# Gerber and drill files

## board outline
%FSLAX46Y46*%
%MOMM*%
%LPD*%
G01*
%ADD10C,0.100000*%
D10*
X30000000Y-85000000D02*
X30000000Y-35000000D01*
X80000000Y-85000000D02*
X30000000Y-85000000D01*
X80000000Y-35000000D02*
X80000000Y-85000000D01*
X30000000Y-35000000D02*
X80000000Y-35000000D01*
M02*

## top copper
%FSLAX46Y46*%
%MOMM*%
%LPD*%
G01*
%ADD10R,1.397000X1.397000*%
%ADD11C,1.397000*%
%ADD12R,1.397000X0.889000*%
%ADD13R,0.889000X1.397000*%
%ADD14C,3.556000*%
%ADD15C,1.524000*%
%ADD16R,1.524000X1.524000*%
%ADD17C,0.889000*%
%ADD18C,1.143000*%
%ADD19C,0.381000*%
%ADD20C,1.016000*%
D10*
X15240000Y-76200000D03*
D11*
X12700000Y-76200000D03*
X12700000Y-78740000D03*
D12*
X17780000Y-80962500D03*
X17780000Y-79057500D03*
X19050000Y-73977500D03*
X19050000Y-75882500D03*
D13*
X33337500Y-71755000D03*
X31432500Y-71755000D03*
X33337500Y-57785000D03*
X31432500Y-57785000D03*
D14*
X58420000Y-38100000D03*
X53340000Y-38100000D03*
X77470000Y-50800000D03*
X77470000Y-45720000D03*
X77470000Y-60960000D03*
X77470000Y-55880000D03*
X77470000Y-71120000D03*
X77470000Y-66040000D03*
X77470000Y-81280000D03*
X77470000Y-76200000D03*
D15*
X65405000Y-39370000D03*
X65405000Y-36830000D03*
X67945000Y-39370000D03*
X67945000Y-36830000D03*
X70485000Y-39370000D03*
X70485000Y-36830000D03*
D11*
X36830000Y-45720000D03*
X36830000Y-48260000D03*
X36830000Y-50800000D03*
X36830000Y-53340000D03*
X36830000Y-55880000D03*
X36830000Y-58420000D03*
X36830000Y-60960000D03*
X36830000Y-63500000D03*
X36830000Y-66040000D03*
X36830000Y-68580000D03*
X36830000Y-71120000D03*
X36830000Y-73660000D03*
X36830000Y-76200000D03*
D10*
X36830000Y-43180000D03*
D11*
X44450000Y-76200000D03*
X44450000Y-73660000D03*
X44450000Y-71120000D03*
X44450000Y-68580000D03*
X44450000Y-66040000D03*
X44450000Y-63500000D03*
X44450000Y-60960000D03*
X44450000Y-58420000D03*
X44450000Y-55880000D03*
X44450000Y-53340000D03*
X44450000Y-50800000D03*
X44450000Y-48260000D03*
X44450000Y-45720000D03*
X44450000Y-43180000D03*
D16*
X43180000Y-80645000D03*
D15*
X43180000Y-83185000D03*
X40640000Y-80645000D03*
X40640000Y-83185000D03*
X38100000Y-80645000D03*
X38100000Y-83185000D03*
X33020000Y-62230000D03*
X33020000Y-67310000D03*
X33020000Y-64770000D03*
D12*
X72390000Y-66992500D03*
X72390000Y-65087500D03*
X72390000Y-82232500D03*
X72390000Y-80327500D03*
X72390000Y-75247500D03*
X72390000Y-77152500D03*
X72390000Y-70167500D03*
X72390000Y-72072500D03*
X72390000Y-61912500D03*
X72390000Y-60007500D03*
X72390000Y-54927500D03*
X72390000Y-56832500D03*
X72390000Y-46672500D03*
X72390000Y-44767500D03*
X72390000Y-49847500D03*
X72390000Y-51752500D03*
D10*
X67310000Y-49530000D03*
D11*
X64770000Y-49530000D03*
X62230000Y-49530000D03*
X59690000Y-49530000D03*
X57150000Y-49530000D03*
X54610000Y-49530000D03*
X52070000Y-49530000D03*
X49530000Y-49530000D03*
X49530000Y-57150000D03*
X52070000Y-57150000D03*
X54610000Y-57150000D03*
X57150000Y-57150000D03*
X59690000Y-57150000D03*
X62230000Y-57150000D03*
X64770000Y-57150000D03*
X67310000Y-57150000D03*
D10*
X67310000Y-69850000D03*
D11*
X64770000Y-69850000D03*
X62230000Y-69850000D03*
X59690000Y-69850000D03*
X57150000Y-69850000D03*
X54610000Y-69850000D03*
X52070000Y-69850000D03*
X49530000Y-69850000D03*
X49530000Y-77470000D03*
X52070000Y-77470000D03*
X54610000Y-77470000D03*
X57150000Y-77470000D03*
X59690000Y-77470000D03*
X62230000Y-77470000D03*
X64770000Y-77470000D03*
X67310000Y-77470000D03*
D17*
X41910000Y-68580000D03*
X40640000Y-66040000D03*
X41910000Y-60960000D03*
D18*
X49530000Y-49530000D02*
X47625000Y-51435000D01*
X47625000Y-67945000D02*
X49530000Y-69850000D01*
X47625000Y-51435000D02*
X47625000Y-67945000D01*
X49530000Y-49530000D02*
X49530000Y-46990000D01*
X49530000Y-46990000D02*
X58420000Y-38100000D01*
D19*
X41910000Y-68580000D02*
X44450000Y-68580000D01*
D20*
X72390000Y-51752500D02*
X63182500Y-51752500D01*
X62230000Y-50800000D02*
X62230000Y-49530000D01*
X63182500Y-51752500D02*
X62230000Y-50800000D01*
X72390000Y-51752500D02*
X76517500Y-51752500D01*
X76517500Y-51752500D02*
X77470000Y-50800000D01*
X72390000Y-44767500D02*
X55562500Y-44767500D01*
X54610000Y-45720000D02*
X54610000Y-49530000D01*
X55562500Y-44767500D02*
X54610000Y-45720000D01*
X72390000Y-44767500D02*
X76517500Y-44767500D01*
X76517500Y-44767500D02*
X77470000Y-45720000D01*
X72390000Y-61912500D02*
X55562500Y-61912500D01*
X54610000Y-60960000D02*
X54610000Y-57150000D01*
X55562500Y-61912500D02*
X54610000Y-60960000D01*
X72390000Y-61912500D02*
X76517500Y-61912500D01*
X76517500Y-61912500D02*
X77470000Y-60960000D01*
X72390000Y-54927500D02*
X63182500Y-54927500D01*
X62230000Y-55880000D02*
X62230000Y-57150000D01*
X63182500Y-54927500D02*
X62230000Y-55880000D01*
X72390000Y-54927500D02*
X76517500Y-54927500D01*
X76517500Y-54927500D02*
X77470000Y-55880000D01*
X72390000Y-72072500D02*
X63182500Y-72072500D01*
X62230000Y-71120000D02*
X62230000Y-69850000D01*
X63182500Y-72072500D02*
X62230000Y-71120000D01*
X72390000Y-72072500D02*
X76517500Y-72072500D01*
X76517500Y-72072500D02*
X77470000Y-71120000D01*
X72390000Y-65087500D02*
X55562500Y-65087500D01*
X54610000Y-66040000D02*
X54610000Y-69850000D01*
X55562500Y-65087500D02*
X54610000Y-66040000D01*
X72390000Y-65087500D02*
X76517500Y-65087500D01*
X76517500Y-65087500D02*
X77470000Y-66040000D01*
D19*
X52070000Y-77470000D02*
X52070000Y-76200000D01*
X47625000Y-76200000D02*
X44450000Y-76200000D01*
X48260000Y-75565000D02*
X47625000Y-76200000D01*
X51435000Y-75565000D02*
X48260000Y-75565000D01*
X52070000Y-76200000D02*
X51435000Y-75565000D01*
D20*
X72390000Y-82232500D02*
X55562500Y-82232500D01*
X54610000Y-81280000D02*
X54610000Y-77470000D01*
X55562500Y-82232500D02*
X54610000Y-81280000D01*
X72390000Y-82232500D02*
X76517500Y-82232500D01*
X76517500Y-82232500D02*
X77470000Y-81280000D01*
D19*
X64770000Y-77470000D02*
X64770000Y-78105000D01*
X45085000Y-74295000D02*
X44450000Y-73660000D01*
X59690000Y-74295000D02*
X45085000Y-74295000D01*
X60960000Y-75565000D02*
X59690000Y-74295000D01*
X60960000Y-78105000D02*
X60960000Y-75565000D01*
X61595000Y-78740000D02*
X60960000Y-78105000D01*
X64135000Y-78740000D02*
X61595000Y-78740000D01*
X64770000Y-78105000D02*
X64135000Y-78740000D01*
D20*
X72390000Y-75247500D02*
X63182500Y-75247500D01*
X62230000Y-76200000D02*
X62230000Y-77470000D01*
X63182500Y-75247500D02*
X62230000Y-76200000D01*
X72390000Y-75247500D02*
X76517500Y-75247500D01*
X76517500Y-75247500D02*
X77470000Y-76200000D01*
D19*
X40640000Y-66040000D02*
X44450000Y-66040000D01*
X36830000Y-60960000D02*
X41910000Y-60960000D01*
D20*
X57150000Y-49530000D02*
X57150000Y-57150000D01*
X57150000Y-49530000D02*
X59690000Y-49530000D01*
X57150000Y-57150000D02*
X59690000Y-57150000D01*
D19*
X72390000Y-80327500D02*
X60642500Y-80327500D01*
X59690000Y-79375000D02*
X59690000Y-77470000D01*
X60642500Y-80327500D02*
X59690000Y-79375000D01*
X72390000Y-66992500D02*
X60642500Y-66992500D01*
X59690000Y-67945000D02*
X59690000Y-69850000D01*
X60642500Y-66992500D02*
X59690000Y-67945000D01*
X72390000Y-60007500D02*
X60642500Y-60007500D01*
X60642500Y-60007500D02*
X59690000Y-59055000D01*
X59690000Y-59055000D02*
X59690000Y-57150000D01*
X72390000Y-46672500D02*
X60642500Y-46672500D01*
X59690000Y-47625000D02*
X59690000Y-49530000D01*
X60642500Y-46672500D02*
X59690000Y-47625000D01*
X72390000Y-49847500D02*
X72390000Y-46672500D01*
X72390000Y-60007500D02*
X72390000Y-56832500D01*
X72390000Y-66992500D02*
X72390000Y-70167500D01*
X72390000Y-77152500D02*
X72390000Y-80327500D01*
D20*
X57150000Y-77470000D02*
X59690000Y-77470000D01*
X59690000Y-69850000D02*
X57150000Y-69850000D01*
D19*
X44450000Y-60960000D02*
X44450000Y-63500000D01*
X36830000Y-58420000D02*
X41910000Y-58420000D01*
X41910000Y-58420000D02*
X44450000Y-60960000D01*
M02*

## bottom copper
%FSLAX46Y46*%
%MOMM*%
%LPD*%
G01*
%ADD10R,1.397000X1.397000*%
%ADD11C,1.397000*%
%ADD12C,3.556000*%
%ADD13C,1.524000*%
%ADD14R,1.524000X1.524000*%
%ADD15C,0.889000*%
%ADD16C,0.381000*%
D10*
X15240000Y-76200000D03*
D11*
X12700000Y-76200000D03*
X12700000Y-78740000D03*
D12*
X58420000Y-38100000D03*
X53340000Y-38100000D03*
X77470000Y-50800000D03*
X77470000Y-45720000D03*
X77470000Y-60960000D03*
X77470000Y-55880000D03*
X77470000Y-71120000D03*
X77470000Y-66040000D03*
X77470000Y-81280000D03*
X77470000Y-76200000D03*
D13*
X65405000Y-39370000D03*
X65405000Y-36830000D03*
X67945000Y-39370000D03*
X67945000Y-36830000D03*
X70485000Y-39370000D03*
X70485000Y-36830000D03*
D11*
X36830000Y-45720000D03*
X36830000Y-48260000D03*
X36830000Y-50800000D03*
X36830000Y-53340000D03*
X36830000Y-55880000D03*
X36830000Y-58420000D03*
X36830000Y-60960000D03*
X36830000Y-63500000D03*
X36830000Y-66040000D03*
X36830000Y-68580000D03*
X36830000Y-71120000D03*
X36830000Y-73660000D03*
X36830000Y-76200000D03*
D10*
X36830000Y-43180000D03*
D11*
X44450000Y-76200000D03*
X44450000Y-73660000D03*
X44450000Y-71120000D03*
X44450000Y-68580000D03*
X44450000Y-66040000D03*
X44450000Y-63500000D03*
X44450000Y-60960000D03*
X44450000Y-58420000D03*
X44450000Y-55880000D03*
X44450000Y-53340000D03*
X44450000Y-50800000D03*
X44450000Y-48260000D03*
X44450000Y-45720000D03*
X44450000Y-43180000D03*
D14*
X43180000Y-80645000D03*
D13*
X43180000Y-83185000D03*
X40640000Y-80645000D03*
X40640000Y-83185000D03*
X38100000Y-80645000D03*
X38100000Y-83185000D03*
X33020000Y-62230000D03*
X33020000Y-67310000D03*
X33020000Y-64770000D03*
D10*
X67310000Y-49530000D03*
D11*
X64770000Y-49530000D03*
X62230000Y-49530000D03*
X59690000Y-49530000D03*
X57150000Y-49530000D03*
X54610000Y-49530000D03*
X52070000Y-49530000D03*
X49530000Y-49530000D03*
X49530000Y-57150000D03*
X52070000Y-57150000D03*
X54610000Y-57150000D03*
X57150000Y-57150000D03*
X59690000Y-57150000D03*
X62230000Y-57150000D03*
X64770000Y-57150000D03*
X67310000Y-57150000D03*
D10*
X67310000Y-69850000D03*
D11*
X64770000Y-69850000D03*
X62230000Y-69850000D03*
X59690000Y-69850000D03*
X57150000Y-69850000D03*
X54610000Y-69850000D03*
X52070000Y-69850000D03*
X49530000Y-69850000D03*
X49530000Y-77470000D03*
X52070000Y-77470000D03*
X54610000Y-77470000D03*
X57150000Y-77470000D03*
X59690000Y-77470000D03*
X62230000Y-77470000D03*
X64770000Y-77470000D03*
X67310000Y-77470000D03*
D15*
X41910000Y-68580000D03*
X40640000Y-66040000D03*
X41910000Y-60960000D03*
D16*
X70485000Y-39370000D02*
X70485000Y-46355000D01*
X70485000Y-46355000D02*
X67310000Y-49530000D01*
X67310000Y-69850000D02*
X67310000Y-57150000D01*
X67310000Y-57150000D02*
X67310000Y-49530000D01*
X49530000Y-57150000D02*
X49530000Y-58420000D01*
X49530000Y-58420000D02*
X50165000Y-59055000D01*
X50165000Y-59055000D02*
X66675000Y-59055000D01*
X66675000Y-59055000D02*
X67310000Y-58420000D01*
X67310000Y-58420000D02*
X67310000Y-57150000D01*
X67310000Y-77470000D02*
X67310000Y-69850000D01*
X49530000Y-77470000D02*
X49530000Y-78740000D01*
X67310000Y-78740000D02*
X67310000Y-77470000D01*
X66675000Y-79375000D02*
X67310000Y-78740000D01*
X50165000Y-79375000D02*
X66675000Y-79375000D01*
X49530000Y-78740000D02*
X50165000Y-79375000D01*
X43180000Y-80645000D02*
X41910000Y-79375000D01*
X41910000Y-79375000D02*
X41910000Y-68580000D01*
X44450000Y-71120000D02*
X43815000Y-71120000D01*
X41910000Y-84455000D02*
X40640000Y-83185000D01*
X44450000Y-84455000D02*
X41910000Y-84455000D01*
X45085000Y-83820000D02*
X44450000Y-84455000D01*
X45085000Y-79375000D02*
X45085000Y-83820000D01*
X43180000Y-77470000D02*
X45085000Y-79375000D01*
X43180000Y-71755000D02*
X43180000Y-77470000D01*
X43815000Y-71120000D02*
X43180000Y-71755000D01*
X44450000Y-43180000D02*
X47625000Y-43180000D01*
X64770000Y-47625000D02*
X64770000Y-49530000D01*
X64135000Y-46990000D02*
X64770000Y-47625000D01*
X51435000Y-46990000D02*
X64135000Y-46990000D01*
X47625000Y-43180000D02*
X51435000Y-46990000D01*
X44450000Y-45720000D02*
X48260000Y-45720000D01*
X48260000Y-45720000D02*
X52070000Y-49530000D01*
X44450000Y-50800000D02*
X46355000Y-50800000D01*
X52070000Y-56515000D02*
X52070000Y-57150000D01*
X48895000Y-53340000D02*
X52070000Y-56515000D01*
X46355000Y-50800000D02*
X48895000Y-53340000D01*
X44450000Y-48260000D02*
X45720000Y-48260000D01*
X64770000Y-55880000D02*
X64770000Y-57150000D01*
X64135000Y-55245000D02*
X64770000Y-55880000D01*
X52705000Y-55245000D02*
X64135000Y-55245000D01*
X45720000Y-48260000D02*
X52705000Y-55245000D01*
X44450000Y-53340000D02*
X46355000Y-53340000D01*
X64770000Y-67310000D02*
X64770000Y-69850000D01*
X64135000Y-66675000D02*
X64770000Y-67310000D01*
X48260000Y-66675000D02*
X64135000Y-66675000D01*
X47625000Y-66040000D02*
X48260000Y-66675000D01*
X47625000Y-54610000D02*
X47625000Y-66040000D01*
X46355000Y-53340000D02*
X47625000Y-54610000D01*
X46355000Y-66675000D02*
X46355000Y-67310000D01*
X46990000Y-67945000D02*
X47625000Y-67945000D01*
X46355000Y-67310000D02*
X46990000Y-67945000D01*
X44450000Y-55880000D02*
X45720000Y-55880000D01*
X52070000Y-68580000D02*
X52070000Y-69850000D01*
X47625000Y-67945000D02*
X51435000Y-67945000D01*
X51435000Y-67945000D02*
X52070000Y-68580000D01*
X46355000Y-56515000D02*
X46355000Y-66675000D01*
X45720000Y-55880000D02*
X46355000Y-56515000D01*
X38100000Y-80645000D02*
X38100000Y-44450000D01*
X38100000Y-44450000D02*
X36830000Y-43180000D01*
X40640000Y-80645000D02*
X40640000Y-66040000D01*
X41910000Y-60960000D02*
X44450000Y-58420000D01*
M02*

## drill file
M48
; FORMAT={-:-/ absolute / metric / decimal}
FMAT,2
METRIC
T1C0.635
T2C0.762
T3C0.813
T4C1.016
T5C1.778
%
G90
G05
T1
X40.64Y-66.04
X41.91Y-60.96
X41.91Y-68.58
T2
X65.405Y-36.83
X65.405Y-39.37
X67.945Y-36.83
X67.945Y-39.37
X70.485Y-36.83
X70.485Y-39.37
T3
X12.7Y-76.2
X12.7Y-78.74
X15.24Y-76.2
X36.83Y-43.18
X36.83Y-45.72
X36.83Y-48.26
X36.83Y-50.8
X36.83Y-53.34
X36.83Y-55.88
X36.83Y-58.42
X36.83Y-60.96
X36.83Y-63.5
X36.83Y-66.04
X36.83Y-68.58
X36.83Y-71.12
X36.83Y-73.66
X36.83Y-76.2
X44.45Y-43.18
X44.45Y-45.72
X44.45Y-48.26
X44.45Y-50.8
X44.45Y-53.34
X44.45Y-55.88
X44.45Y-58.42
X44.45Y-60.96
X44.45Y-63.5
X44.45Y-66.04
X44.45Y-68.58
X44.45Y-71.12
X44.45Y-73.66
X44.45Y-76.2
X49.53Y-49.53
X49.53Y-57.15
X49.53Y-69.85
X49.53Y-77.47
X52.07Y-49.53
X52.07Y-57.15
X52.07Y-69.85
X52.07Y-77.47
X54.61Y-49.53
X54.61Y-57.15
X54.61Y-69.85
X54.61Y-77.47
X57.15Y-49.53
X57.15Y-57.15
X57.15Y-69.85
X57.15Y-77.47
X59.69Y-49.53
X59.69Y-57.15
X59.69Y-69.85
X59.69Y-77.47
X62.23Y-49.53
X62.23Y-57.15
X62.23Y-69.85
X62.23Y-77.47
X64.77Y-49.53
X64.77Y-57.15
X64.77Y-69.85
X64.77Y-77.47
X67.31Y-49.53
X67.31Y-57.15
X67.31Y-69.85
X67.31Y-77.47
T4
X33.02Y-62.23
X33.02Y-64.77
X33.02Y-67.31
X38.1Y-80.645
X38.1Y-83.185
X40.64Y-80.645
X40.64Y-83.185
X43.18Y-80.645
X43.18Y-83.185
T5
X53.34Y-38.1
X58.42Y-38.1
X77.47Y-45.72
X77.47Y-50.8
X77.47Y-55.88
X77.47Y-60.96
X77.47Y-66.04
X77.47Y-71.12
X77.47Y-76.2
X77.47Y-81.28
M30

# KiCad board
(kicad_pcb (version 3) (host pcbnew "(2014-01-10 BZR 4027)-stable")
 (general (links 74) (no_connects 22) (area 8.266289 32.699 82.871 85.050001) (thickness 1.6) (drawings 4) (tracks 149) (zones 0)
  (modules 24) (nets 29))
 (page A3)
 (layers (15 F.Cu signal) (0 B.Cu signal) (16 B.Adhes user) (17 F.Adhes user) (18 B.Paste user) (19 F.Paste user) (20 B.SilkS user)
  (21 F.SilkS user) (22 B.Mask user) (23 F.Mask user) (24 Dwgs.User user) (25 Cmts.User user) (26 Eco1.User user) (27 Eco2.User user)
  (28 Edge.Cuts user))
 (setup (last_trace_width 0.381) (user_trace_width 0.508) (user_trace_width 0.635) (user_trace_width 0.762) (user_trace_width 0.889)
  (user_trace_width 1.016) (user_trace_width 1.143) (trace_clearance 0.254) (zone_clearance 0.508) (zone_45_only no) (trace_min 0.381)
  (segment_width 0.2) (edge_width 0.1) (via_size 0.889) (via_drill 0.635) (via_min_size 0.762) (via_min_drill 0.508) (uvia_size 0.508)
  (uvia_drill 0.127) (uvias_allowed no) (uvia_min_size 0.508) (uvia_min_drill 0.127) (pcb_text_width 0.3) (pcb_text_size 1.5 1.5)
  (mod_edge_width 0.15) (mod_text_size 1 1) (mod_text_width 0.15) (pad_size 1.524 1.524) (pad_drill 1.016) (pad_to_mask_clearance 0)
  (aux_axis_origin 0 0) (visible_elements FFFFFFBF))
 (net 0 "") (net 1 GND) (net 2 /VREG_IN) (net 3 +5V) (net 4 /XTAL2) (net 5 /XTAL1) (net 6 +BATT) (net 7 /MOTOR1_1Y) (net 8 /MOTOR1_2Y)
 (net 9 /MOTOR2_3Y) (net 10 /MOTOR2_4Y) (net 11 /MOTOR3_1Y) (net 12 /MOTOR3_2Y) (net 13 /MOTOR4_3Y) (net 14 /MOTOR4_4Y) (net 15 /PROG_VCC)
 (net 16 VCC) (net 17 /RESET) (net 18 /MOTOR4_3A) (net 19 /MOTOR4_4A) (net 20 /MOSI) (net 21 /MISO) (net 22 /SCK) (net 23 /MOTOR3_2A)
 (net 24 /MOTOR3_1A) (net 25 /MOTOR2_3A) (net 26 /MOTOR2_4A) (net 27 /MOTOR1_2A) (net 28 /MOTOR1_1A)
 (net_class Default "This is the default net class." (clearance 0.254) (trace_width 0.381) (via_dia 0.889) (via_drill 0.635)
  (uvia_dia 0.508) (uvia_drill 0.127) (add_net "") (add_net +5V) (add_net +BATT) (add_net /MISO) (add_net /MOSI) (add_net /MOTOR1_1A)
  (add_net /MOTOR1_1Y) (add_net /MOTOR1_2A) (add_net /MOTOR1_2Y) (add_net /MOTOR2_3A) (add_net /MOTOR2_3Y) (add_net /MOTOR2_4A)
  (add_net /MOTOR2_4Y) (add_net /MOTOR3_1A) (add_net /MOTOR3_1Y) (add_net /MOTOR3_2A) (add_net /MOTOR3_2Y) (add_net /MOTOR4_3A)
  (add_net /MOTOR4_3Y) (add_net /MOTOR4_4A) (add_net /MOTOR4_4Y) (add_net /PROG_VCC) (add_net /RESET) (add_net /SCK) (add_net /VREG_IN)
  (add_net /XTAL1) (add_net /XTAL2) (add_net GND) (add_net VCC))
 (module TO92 (layer F.Cu) (at 13.97 77.47)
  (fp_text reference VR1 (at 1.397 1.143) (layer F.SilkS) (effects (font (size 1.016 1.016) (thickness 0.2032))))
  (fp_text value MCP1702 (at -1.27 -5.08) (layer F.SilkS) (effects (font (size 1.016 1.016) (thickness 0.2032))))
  (pad 1 thru_hole rect (at 1.27 -1.27) (size 1.397 1.397) (drill 0.8128) (layers *.Cu *.Mask F.SilkS) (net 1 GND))
  (pad 2 thru_hole circle (at -1.27 -1.27) (size 1.397 1.397) (drill 0.8128) (layers *.Cu *.Mask F.SilkS) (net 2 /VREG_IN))
  (pad 3 thru_hole circle (at -1.27 1.27) (size 1.397 1.397) (drill 0.8128) (layers *.Cu *.Mask F.SilkS) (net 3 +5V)))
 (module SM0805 (layer F.Cu) (at 17.78 80.01 90)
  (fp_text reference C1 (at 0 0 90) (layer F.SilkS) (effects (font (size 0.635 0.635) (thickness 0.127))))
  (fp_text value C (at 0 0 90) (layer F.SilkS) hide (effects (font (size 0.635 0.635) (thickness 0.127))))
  (pad 1 smd rect (at -0.9525 0 90) (size 0.889 1.397) (layers F.Cu F.Paste F.Mask) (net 3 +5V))
  (pad 2 smd rect (at 0.9525 0 90) (size 0.889 1.397) (layers F.Cu F.Paste F.Mask) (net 1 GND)))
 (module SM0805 (layer F.Cu) (at 19.05 74.93 270)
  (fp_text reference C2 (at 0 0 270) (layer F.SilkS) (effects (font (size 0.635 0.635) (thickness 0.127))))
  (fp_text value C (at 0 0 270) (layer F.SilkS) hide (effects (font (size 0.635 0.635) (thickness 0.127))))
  (pad 1 smd rect (at -0.9525 0 270) (size 0.889 1.397) (layers F.Cu F.Paste F.Mask) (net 2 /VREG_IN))
  (pad 2 smd rect (at 0.9525 0 270) (size 0.889 1.397) (layers F.Cu F.Paste F.Mask) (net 1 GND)))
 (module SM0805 (layer F.Cu) (at 32.385 71.755 180)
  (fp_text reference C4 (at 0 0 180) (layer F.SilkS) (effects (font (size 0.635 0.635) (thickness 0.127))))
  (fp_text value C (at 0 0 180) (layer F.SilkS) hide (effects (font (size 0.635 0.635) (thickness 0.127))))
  (pad 1 smd rect (at -0.9525 0 180) (size 0.889 1.397) (layers F.Cu F.Paste F.Mask) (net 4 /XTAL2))
  (pad 2 smd rect (at 0.9525 0 180) (size 0.889 1.397) (layers F.Cu F.Paste F.Mask) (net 1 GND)))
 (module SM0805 (layer F.Cu) (at 32.385 57.785 180)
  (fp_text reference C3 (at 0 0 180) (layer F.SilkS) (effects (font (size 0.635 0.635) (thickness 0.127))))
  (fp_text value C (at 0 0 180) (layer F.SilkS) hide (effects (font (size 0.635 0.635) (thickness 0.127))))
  (pad 1 smd rect (at -0.9525 0 180) (size 0.889 1.397) (layers F.Cu F.Paste F.Mask) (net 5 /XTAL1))
  (pad 2 smd rect (at 0.9525 0 180) (size 0.889 1.397) (layers F.Cu F.Paste F.Mask) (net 1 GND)))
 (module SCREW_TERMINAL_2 (layer F.Cu) (at 55.88 38.1 180)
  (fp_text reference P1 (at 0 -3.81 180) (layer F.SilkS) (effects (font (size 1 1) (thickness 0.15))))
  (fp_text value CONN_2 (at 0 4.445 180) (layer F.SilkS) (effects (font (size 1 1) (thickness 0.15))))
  (pad 1 thru_hole circle (at -2.54 0 180) (size 3.556 3.556) (drill 1.778) (layers *.Cu *.Mask F.SilkS) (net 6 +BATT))
  (pad 2 thru_hole circle (at 2.54 0 180) (size 3.556 3.556) (drill 1.778) (layers *.Cu *.Mask F.SilkS) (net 1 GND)))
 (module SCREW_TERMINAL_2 (layer F.Cu) (at 77.47 48.26 90)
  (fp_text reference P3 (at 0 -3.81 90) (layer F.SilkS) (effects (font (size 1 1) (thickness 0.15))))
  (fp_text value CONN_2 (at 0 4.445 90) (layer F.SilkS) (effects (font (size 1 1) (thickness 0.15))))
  (pad 1 thru_hole circle (at -2.54 0 90) (size 3.556 3.556) (drill 1.778) (layers *.Cu *.Mask F.SilkS) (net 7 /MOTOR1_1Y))
  (pad 2 thru_hole circle (at 2.54 0 90) (size 3.556 3.556) (drill 1.778) (layers *.Cu *.Mask F.SilkS) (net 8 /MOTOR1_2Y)))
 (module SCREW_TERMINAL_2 (layer F.Cu) (at 77.47 58.42 90)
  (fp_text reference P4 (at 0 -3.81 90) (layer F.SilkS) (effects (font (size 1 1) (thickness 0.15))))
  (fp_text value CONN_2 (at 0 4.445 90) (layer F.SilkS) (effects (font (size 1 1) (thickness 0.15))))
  (pad 1 thru_hole circle (at -2.54 0 90) (size 3.556 3.556) (drill 1.778) (layers *.Cu *.Mask F.SilkS) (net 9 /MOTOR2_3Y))
  (pad 2 thru_hole circle (at 2.54 0 90) (size 3.556 3.556) (drill 1.778) (layers *.Cu *.Mask F.SilkS) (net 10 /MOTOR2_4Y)))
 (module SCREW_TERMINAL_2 (layer F.Cu) (at 77.47 68.58 90)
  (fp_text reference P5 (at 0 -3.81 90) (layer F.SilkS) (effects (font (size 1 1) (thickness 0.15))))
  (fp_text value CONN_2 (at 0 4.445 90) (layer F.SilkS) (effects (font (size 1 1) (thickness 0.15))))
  (pad 1 thru_hole circle (at -2.54 0 90) (size 3.556 3.556) (drill 1.778) (layers *.Cu *.Mask F.SilkS) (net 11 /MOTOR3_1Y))
  (pad 2 thru_hole circle (at 2.54 0 90) (size 3.556 3.556) (drill 1.778) (layers *.Cu *.Mask F.SilkS) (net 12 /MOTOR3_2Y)))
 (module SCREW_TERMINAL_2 (layer F.Cu) (at 77.47 78.74 90)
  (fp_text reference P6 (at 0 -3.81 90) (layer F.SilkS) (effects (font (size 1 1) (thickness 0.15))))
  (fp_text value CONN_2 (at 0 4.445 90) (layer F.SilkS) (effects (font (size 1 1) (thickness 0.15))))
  (pad 1 thru_hole circle (at -2.54 0 90) (size 3.556 3.556) (drill 1.778) (layers *.Cu *.Mask F.SilkS) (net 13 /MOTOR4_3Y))
  (pad 2 thru_hole circle (at 2.54 0 90) (size 3.556 3.556) (drill 1.778) (layers *.Cu *.Mask F.SilkS) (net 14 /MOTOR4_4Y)))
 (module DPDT (layer F.Cu) (at 67.945 38.1)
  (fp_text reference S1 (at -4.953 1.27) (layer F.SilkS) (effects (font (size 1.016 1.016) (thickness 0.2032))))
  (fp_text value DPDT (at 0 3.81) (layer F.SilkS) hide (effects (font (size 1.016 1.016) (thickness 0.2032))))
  (pad 4 thru_hole circle (at -2.54 1.27) (size 1.524 1.524) (drill 0.762) (layers *.Cu *.Mask F.SilkS) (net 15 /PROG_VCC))
  (pad 1 thru_hole circle (at -2.54 -1.27) (size 1.524 1.524) (drill 0.762) (layers *.Cu *.Mask F.SilkS) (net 2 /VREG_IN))
  (pad 5 thru_hole circle (at 0 1.27) (size 1.524 1.524) (drill 0.762) (layers *.Cu *.Mask F.SilkS) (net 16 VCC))
  (pad 2 thru_hole circle (at 0 -1.27) (size 1.524 1.524) (drill 0.762) (layers *.Cu *.Mask F.SilkS) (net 6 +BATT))
  (pad 6 thru_hole circle (at 2.54 1.27) (size 1.524 1.524) (drill 0.762) (layers *.Cu *.Mask F.SilkS) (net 3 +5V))
  (pad 3 thru_hole circle (at 2.54 -1.27) (size 1.524 1.524) (drill 0.762) (layers *.Cu *.Mask F.SilkS)))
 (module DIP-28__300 (layer F.Cu) (at 40.64 59.69 270)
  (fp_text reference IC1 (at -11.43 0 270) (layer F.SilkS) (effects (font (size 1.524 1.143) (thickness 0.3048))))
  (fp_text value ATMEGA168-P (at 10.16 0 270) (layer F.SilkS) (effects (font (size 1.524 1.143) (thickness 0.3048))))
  (pad 2 thru_hole circle (at -13.97 3.81 270) (size 1.397 1.397) (drill 0.8128) (layers *.Cu *.Mask F.SilkS))
  (pad 3 thru_hole circle (at -11.43 3.81 270) (size 1.397 1.397) (drill 0.8128) (layers *.Cu *.Mask F.SilkS))
  (pad 4 thru_hole circle (at -8.89 3.81 270) (size 1.397 1.397) (drill 0.8128) (layers *.Cu *.Mask F.SilkS))
  (pad 5 thru_hole circle (at -6.35 3.81 270) (size 1.397 1.397) (drill 0.8128) (layers *.Cu *.Mask F.SilkS))
  (pad 6 thru_hole circle (at -3.81 3.81 270) (size 1.397 1.397) (drill 0.8128) (layers *.Cu *.Mask F.SilkS))
  (pad 7 thru_hole circle (at -1.27 3.81 270) (size 1.397 1.397) (drill 0.8128) (layers *.Cu *.Mask F.SilkS) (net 16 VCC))
  (pad 8 thru_hole circle (at 1.27 3.81 270) (size 1.397 1.397) (drill 0.8128) (layers *.Cu *.Mask F.SilkS) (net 1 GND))
  (pad 9 thru_hole circle (at 3.81 3.81 270) (size 1.397 1.397) (drill 0.8128) (layers *.Cu *.Mask F.SilkS) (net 5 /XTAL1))
  (pad 10 thru_hole circle (at 6.35 3.81 270) (size 1.397 1.397) (drill 0.8128) (layers *.Cu *.Mask F.SilkS) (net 4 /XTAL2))
  (pad 11 thru_hole circle (at 8.89 3.81 270) (size 1.397 1.397) (drill 0.8128) (layers *.Cu *.Mask F.SilkS))
  (pad 12 thru_hole circle (at 11.43 3.81 270) (size 1.397 1.397) (drill 0.8128) (layers *.Cu *.Mask F.SilkS))
  (pad 13 thru_hole circle (at 13.97 3.81 270) (size 1.397 1.397) (drill 0.8128) (layers *.Cu *.Mask F.SilkS))
  (pad 14 thru_hole circle (at 16.51 3.81 270) (size 1.397 1.397) (drill 0.8128) (layers *.Cu *.Mask F.SilkS))
  (pad 1 thru_hole rect (at -16.51 3.81 270) (size 1.397 1.397) (drill 0.8128) (layers *.Cu *.Mask F.SilkS) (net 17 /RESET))
  (pad 15 thru_hole circle (at 16.51 -3.81 270) (size 1.397 1.397) (drill 0.8128) (layers *.Cu *.Mask F.SilkS) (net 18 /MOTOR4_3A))
  (pad 16 thru_hole circle (at 13.97 -3.81 270) (size 1.397 1.397) (drill 0.8128) (layers *.Cu *.Mask F.SilkS) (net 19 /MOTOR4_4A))
  (pad 17 thru_hole circle (at 11.43 -3.81 270) (size 1.397 1.397) (drill 0.8128) (layers *.Cu *.Mask F.SilkS) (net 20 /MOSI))
  (pad 18 thru_hole circle (at 8.89 -3.81 270) (size 1.397 1.397) (drill 0.8128) (layers *.Cu *.Mask F.SilkS) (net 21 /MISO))
  (pad 19 thru_hole circle (at 6.35 -3.81 270) (size 1.397 1.397) (drill 0.8128) (layers *.Cu *.Mask F.SilkS) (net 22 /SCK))
  (pad 20 thru_hole circle (at 3.81 -3.81 270) (size 1.397 1.397) (drill 0.8128) (layers *.Cu *.Mask F.SilkS) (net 16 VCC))
  (pad 21 thru_hole circle (at 1.27 -3.81 270) (size 1.397 1.397) (drill 0.8128) (layers *.Cu *.Mask F.SilkS) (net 16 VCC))
  (pad 22 thru_hole circle (at -1.27 -3.81 270) (size 1.397 1.397) (drill 0.8128) (layers *.Cu *.Mask F.SilkS) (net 1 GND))
  (pad 23 thru_hole circle (at -3.81 -3.81 270) (size 1.397 1.397) (drill 0.8128) (layers *.Cu *.Mask F.SilkS) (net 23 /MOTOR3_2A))
  (pad 24 thru_hole circle (at -6.35 -3.81 270) (size 1.397 1.397) (drill 0.8128) (layers *.Cu *.Mask F.SilkS) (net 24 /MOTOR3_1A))
  (pad 25 thru_hole circle (at -8.89 -3.81 270) (size 1.397 1.397) (drill 0.8128) (layers *.Cu *.Mask F.SilkS) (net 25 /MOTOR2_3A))
  (pad 26 thru_hole circle (at -11.43 -3.81 270) (size 1.397 1.397) (drill 0.8128) (layers *.Cu *.Mask F.SilkS) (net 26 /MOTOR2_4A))
  (pad 27 thru_hole circle (at -13.97 -3.81 270) (size 1.397 1.397) (drill 0.8128) (layers *.Cu *.Mask F.SilkS) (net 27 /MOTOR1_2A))
  (pad 28 thru_hole circle (at -16.51 -3.81 270) (size 1.397 1.397) (drill 0.8128) (layers *.Cu *.Mask F.SilkS) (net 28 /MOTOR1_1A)))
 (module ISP (layer F.Cu) (at 40.64 81.915 180)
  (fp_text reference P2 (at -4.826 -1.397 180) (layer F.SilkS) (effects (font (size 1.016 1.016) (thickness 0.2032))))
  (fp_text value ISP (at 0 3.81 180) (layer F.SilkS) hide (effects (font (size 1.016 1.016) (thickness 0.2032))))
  (pad 1 thru_hole rect (at -2.54 1.27 180) (size 1.524 1.524) (drill 1.016) (layers *.Cu *.Mask F.SilkS) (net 21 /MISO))
  (pad 2 thru_hole circle (at -2.54 -1.27 180) (size 1.524 1.524) (drill 1.016) (layers *.Cu *.Mask F.SilkS) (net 15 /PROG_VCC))
  (pad 3 thru_hole circle (at 0 1.27 180) (size 1.524 1.524) (drill 1.016) (layers *.Cu *.Mask F.SilkS) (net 22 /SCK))
  (pad 4 thru_hole circle (at 0 -1.27 180) (size 1.524 1.524) (drill 1.016) (layers *.Cu *.Mask F.SilkS) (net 20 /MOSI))
  (pad 5 thru_hole circle (at 2.54 1.27 180) (size 1.524 1.524) (drill 1.016) (layers *.Cu *.Mask F.SilkS) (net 17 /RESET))
  (pad 6 thru_hole circle (at 2.54 -1.27 180) (size 1.524 1.524) (drill 1.016) (layers *.Cu *.Mask F.SilkS) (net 1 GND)))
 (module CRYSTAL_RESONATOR (layer F.Cu) (at 33.02 64.77 270)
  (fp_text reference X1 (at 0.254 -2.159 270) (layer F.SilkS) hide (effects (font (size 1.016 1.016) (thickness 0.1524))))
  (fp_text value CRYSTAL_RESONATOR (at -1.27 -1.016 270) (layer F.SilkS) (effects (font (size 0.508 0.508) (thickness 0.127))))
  (pad 1 thru_hole circle (at -2.54 0 270) (size 1.524 1.524) (drill 1.016) (layers *.Cu *.Mask F.SilkS) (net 5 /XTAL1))
  (pad 2 thru_hole circle (at 2.54 0 270) (size 1.524 1.524) (drill 1.016) (layers *.Cu *.Mask F.SilkS) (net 4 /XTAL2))
  (pad 3 thru_hole circle (at 0 0 270) (size 1.524 1.524) (drill 1.016) (layers *.Cu *.Mask F.SilkS) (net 1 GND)))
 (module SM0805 (layer F.Cu) (at 72.39 66.04 90)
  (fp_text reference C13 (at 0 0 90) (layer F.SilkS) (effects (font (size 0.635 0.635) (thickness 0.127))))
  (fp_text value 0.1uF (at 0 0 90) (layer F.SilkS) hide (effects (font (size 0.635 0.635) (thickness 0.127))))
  (pad 1 smd rect (at -0.9525 0 90) (size 0.889 1.397) (layers F.Cu F.Paste F.Mask) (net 1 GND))
  (pad 2 smd rect (at 0.9525 0 90) (size 0.889 1.397) (layers F.Cu F.Paste F.Mask) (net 12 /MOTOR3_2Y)))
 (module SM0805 (layer F.Cu) (at 72.39 81.28 90)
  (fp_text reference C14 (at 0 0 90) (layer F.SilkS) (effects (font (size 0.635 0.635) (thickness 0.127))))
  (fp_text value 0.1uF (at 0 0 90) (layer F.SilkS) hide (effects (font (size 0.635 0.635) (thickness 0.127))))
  (pad 1 smd rect (at -0.9525 0 90) (size 0.889 1.397) (layers F.Cu F.Paste F.Mask) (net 13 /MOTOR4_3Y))
  (pad 2 smd rect (at 0.9525 0 90) (size 0.889 1.397) (layers F.Cu F.Paste F.Mask) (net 1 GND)))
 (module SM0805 (layer F.Cu) (at 72.39 76.2 270)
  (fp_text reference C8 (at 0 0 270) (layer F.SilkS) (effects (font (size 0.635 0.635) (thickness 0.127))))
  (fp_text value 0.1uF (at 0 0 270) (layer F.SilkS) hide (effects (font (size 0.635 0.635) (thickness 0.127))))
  (pad 1 smd rect (at -0.9525 0 270) (size 0.889 1.397) (layers F.Cu F.Paste F.Mask) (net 14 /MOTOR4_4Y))
  (pad 2 smd rect (at 0.9525 0 270) (size 0.889 1.397) (layers F.Cu F.Paste F.Mask) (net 1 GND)))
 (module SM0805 (layer F.Cu) (at 72.39 71.12 270)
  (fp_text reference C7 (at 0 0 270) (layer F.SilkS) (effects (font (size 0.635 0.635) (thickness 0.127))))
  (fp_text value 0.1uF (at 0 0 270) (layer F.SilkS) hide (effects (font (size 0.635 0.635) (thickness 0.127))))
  (pad 1 smd rect (at -0.9525 0 270) (size 0.889 1.397) (layers F.Cu F.Paste F.Mask) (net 1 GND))
  (pad 2 smd rect (at 0.9525 0 270) (size 0.889 1.397) (layers F.Cu F.Paste F.Mask) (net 11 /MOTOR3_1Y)))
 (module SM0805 (layer F.Cu) (at 72.39 60.96 90)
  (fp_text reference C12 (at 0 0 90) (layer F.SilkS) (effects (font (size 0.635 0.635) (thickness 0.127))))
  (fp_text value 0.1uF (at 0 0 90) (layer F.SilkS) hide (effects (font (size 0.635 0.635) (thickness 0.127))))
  (pad 1 smd rect (at -0.9525 0 90) (size 0.889 1.397) (layers F.Cu F.Paste F.Mask) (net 9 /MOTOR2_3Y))
  (pad 2 smd rect (at 0.9525 0 90) (size 0.889 1.397) (layers F.Cu F.Paste F.Mask) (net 1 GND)))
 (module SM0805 (layer F.Cu) (at 72.39 55.88 270)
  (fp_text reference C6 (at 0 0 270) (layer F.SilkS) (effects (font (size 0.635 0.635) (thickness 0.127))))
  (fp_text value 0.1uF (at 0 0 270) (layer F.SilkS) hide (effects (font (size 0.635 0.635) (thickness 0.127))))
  (pad 1 smd rect (at -0.9525 0 270) (size 0.889 1.397) (layers F.Cu F.Paste F.Mask) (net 10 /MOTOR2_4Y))
  (pad 2 smd rect (at 0.9525 0 270) (size 0.889 1.397) (layers F.Cu F.Paste F.Mask) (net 1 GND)))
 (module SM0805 (layer F.Cu) (at 72.39 45.72 90)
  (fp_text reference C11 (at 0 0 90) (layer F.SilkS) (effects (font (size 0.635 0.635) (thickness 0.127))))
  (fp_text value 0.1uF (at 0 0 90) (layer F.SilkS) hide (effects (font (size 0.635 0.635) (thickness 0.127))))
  (pad 1 smd rect (at -0.9525 0 90) (size 0.889 1.397) (layers F.Cu F.Paste F.Mask) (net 1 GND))
  (pad 2 smd rect (at 0.9525 0 90) (size 0.889 1.397) (layers F.Cu F.Paste F.Mask) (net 8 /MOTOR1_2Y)))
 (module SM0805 (layer F.Cu) (at 72.39 50.8 270)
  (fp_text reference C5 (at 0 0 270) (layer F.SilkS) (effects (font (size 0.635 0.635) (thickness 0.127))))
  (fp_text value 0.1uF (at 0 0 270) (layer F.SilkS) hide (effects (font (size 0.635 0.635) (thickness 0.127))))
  (pad 1 smd rect (at -0.9525 0 270) (size 0.889 1.397) (layers F.Cu F.Paste F.Mask) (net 1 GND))
  (pad 2 smd rect (at 0.9525 0 270) (size 0.889 1.397) (layers F.Cu F.Paste F.Mask) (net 7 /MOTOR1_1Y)))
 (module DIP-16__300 (layer F.Cu) (at 58.42 53.34 180)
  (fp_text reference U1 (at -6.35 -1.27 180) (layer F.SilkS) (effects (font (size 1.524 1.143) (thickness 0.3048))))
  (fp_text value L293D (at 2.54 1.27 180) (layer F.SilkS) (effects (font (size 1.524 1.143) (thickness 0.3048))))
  (pad 1 thru_hole rect (at -8.89 3.81 180) (size 1.397 1.397) (drill 0.8128) (layers *.Cu *.Mask F.SilkS) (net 3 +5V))
  (pad 2 thru_hole circle (at -6.35 3.81 180) (size 1.397 1.397) (drill 0.8128) (layers *.Cu *.Mask F.SilkS) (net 28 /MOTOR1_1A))
  (pad 3 thru_hole circle (at -3.81 3.81 180) (size 1.397 1.397) (drill 0.8128) (layers *.Cu *.Mask F.SilkS) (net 7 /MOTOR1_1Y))
  (pad 4 thru_hole circle (at -1.27 3.81 180) (size 1.397 1.397) (drill 0.8128) (layers *.Cu *.Mask F.SilkS) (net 1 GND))
  (pad 5 thru_hole circle (at 1.27 3.81 180) (size 1.397 1.397) (drill 0.8128) (layers *.Cu *.Mask F.SilkS) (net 1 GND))
  (pad 6 thru_hole circle (at 3.81 3.81 180) (size 1.397 1.397) (drill 0.8128) (layers *.Cu *.Mask F.SilkS) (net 8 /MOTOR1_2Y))
  (pad 7 thru_hole circle (at 6.35 3.81 180) (size 1.397 1.397) (drill 0.8128) (layers *.Cu *.Mask F.SilkS) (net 27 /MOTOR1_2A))
  (pad 8 thru_hole circle (at 8.89 3.81 180) (size 1.397 1.397) (drill 0.8128) (layers *.Cu *.Mask F.SilkS) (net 6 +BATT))
  (pad 9 thru_hole circle (at 8.89 -3.81 180) (size 1.397 1.397) (drill 0.8128) (layers *.Cu *.Mask F.SilkS) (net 3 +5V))
  (pad 10 thru_hole circle (at 6.35 -3.81 180) (size 1.397 1.397) (drill 0.8128) (layers *.Cu *.Mask F.SilkS) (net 25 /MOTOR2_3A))
  (pad 11 thru_hole circle (at 3.81 -3.81 180) (size 1.397 1.397) (drill 0.8128) (layers *.Cu *.Mask F.SilkS) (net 9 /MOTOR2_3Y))
  (pad 12 thru_hole circle (at 1.27 -3.81 180) (size 1.397 1.397) (drill 0.8128) (layers *.Cu *.Mask F.SilkS) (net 1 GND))
  (pad 13 thru_hole circle (at -1.27 -3.81 180) (size 1.397 1.397) (drill 0.8128) (layers *.Cu *.Mask F.SilkS) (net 1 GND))
  (pad 14 thru_hole circle (at -3.81 -3.81 180) (size 1.397 1.397) (drill 0.8128) (layers *.Cu *.Mask F.SilkS) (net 10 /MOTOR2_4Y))
  (pad 15 thru_hole circle (at -6.35 -3.81 180) (size 1.397 1.397) (drill 0.8128) (layers *.Cu *.Mask F.SilkS) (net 26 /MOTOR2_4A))
  (pad 16 thru_hole circle (at -8.89 -3.81 180) (size 1.397 1.397) (drill 0.8128) (layers *.Cu *.Mask F.SilkS) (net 3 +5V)))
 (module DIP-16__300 (layer F.Cu) (at 58.42 73.66 180)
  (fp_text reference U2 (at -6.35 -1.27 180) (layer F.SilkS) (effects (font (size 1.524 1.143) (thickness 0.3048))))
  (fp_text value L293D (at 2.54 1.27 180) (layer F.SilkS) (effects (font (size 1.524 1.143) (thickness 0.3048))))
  (pad 1 thru_hole rect (at -8.89 3.81 180) (size 1.397 1.397) (drill 0.8128) (layers *.Cu *.Mask F.SilkS) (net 3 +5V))
  (pad 2 thru_hole circle (at -6.35 3.81 180) (size 1.397 1.397) (drill 0.8128) (layers *.Cu *.Mask F.SilkS) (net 24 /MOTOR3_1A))
  (pad 3 thru_hole circle (at -3.81 3.81 180) (size 1.397 1.397) (drill 0.8128) (layers *.Cu *.Mask F.SilkS) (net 11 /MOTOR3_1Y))
  (pad 4 thru_hole circle (at -1.27 3.81 180) (size 1.397 1.397) (drill 0.8128) (layers *.Cu *.Mask F.SilkS) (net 1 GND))
  (pad 5 thru_hole circle (at 1.27 3.81 180) (size 1.397 1.397) (drill 0.8128) (layers *.Cu *.Mask F.SilkS) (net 1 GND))
  (pad 6 thru_hole circle (at 3.81 3.81 180) (size 1.397 1.397) (drill 0.8128) (layers *.Cu *.Mask F.SilkS) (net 12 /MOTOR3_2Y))
  (pad 7 thru_hole circle (at 6.35 3.81 180) (size 1.397 1.397) (drill 0.8128) (layers *.Cu *.Mask F.SilkS) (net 23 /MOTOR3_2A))
  (pad 8 thru_hole circle (at 8.89 3.81 180) (size 1.397 1.397) (drill 0.8128) (layers *.Cu *.Mask F.SilkS) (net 6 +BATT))
  (pad 9 thru_hole circle (at 8.89 -3.81 180) (size 1.397 1.397) (drill 0.8128) (layers *.Cu *.Mask F.SilkS) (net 3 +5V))
  (pad 10 thru_hole circle (at 6.35 -3.81 180) (size 1.397 1.397) (drill 0.8128) (layers *.Cu *.Mask F.SilkS) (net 18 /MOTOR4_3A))
  (pad 11 thru_hole circle (at 3.81 -3.81 180) (size 1.397 1.397) (drill 0.8128) (layers *.Cu *.Mask F.SilkS) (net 13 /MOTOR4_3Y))
  (pad 12 thru_hole circle (at 1.27 -3.81 180) (size 1.397 1.397) (drill 0.8128) (layers *.Cu *.Mask F.SilkS) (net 1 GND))
  (pad 13 thru_hole circle (at -1.27 -3.81 180) (size 1.397 1.397) (drill 0.8128) (layers *.Cu *.Mask F.SilkS) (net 1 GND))
  (pad 14 thru_hole circle (at -3.81 -3.81 180) (size 1.397 1.397) (drill 0.8128) (layers *.Cu *.Mask F.SilkS) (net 14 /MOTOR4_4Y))
  (pad 15 thru_hole circle (at -6.35 -3.81 180) (size 1.397 1.397) (drill 0.8128) (layers *.Cu *.Mask F.SilkS) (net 19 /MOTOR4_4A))
  (pad 16 thru_hole circle (at -8.89 -3.81 180) (size 1.397 1.397) (drill 0.8128) (layers *.Cu *.Mask F.SilkS) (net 3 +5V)))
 (gr_line (start 30 85) (end 30 35) (angle 90) (layer Edge.Cuts) (width 0.1))
 (gr_line (start 80 85) (end 30 85) (angle 90) (layer Edge.Cuts) (width 0.1))
 (gr_line (start 80 35) (end 80 85) (angle 90) (layer Edge.Cuts) (width 0.1))
 (gr_line (start 30 35) (end 80 35) (angle 90) (layer Edge.Cuts) (width 0.1))
 (segment (start 70.485 39.37) (end 70.485 46.355) (width 0.381) (layer B.Cu) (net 3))
 (segment (start 70.485 46.355) (end 67.31 49.53) (width 0.381) (layer B.Cu) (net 3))
 (segment (start 67.31 69.85) (end 67.31 57.15) (width 0.381) (layer B.Cu) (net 3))
 (segment (start 67.31 57.15) (end 67.31 49.53) (width 0.381) (layer B.Cu) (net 3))
 (segment (start 49.53 57.15) (end 49.53 58.42) (width 0.381) (layer B.Cu) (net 3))
 (segment (start 49.53 58.42) (end 50.165 59.055) (width 0.381) (layer B.Cu) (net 3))
 (segment (start 50.165 59.055) (end 66.675 59.055) (width 0.381) (layer B.Cu) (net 3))
 (segment (start 66.675 59.055) (end 67.31 58.42) (width 0.381) (layer B.Cu) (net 3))
 (segment (start 67.31 58.42) (end 67.31 57.15) (width 0.381) (layer B.Cu) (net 3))
 (segment (start 67.31 77.47) (end 67.31 69.85) (width 0.381) (layer B.Cu) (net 3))
 (segment (start 49.53 77.47) (end 49.53 78.74) (width 0.381) (layer B.Cu) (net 3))
 (segment (start 67.31 78.74) (end 67.31 77.47) (width 0.381) (layer B.Cu) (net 3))
 (segment (start 66.675 79.375) (end 67.31 78.74) (width 0.381) (layer B.Cu) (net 3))
 (segment (start 50.165 79.375) (end 66.675 79.375) (width 0.381) (layer B.Cu) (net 3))
 (segment (start 49.53 78.74) (end 50.165 79.375) (width 0.381) (layer B.Cu) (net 3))
 (segment (start 49.53 49.53) (end 47.625 51.435) (width 1.143) (layer F.Cu) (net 6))
 (segment (start 47.625 67.945) (end 49.53 69.85) (width 1.143) (layer F.Cu) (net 6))
 (segment (start 47.625 51.435) (end 47.625 67.945) (width 1.143) (layer F.Cu) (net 6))
 (segment (start 49.53 49.53) (end 49.53 46.99) (width 1.143) (layer F.Cu) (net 6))
 (segment (start 49.53 46.99) (end 58.42 38.1) (width 1.143) (layer F.Cu) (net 6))
 (segment (start 43.18 80.645) (end 41.91 79.375) (width 0.381) (layer B.Cu) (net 21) (status 400000))
 (segment (start 41.91 68.58) (end 44.45 68.58) (width 0.381) (layer F.Cu) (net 21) (status 800000))
 (via (at 41.91 68.58) (size 0.889) (layers F.Cu B.Cu) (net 21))
 (segment (start 41.91 79.375) (end 41.91 68.58) (width 0.381) (layer B.Cu) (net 21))
 (segment (start 44.45 71.12) (end 43.815 71.12) (width 0.381) (layer B.Cu) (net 20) (status C00000))
 (segment (start 41.91 84.455) (end 40.64 83.185) (width 0.381) (layer B.Cu) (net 20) (status 800000))
 (segment (start 44.45 84.455) (end 41.91 84.455) (width 0.381) (layer B.Cu) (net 20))
 (segment (start 45.085 83.82) (end 44.45 84.455) (width 0.381) (layer B.Cu) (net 20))
 (segment (start 45.085 79.375) (end 45.085 83.82) (width 0.381) (layer B.Cu) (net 20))
 (segment (start 43.18 77.47) (end 45.085 79.375) (width 0.381) (layer B.Cu) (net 20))
 (segment (start 43.18 71.755) (end 43.18 77.47) (width 0.381) (layer B.Cu) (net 20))
 (segment (start 43.815 71.12) (end 43.18 71.755) (width 0.381) (layer B.Cu) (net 20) (status 400000))
 (segment (start 44.45 43.18) (end 47.625 43.18) (width 0.381) (layer B.Cu) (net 28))
 (segment (start 64.77 47.625) (end 64.77 49.53) (width 0.381) (layer B.Cu) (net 28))
 (segment (start 64.135 46.99) (end 64.77 47.625) (width 0.381) (layer B.Cu) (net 28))
 (segment (start 51.435 46.99) (end 64.135 46.99) (width 0.381) (layer B.Cu) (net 28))
 (segment (start 47.625 43.18) (end 51.435 46.99) (width 0.381) (layer B.Cu) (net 28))
 (segment (start 72.39 51.7525) (end 63.1825 51.7525) (width 1.016) (layer F.Cu) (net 7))
 (segment (start 62.23 50.8) (end 62.23 49.53) (width 1.016) (layer F.Cu) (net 7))
 (segment (start 63.1825 51.7525) (end 62.23 50.8) (width 1.016) (layer F.Cu) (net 7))
 (segment (start 72.39 51.7525) (end 76.5175 51.7525) (width 1.016) (layer F.Cu) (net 7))
 (segment (start 76.5175 51.7525) (end 77.47 50.8) (width 1.016) (layer F.Cu) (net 7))
 (segment (start 44.45 45.72) (end 48.26 45.72) (width 0.381) (layer B.Cu) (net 27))
 (segment (start 48.26 45.72) (end 52.07 49.53) (width 0.381) (layer B.Cu) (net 27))
 (segment (start 72.39 44.7675) (end 55.5625 44.7675) (width 1.016) (layer F.Cu) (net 8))
 (segment (start 54.61 45.72) (end 54.61 49.53) (width 1.016) (layer F.Cu) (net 8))
 (segment (start 55.5625 44.7675) (end 54.61 45.72) (width 1.016) (layer F.Cu) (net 8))
 (segment (start 72.39 44.7675) (end 76.5175 44.7675) (width 1.016) (layer F.Cu) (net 8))
 (segment (start 76.5175 44.7675) (end 77.47 45.72) (width 1.016) (layer F.Cu) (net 8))
 (segment (start 44.45 50.8) (end 46.355 50.8) (width 0.381) (layer B.Cu) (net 25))
 (segment (start 52.07 56.515) (end 52.07 57.15) (width 0.381) (layer B.Cu) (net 25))
 (segment (start 48.895 53.34) (end 52.07 56.515) (width 0.381) (layer B.Cu) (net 25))
 (segment (start 46.355 50.8) (end 48.895 53.34) (width 0.381) (layer B.Cu) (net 25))
 (segment (start 72.39 61.9125) (end 55.5625 61.9125) (width 1.016) (layer F.Cu) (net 9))
 (segment (start 54.61 60.96) (end 54.61 57.15) (width 1.016) (layer F.Cu) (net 9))
 (segment (start 55.5625 61.9125) (end 54.61 60.96) (width 1.016) (layer F.Cu) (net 9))
 (segment (start 72.39 61.9125) (end 76.5175 61.9125) (width 1.016) (layer F.Cu) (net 9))
 (segment (start 76.5175 61.9125) (end 77.47 60.96) (width 1.016) (layer F.Cu) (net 9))
 (segment (start 44.45 48.26) (end 45.72 48.26) (width 0.381) (layer B.Cu) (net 26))
 (segment (start 64.77 55.88) (end 64.77 57.15) (width 0.381) (layer B.Cu) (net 26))
 (segment (start 64.135 55.245) (end 64.77 55.88) (width 0.381) (layer B.Cu) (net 26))
 (segment (start 52.705 55.245) (end 64.135 55.245) (width 0.381) (layer B.Cu) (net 26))
 (segment (start 45.72 48.26) (end 52.705 55.245) (width 0.381) (layer B.Cu) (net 26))
 (segment (start 72.39 54.9275) (end 63.1825 54.9275) (width 1.016) (layer F.Cu) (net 10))
 (segment (start 62.23 55.88) (end 62.23 57.15) (width 1.016) (layer F.Cu) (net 10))
 (segment (start 63.1825 54.9275) (end 62.23 55.88) (width 1.016) (layer F.Cu) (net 10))
 (segment (start 72.39 54.9275) (end 76.5175 54.9275) (width 1.016) (layer F.Cu) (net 10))
 (segment (start 76.5175 54.9275) (end 77.47 55.88) (width 1.016) (layer F.Cu) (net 10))
 (segment (start 44.45 53.34) (end 46.355 53.34) (width 0.381) (layer B.Cu) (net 24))
 (segment (start 64.77 67.31) (end 64.77 69.85) (width 0.381) (layer B.Cu) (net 24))
 (segment (start 64.135 66.675) (end 64.77 67.31) (width 0.381) (layer B.Cu) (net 24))
 (segment (start 48.26 66.675) (end 64.135 66.675) (width 0.381) (layer B.Cu) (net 24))
 (segment (start 47.625 66.04) (end 48.26 66.675) (width 0.381) (layer B.Cu) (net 24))
 (segment (start 47.625 54.61) (end 47.625 66.04) (width 0.381) (layer B.Cu) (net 24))
 (segment (start 46.355 53.34) (end 47.625 54.61) (width 0.381) (layer B.Cu) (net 24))
 (segment (start 72.39 72.0725) (end 63.1825 72.0725) (width 1.016) (layer F.Cu) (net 11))
 (segment (start 62.23 71.12) (end 62.23 69.85) (width 1.016) (layer F.Cu) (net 11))
 (segment (start 63.1825 72.0725) (end 62.23 71.12) (width 1.016) (layer F.Cu) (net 11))
 (segment (start 72.39 72.0725) (end 76.5175 72.0725) (width 1.016) (layer F.Cu) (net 11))
 (segment (start 76.5175 72.0725) (end 77.47 71.12) (width 1.016) (layer F.Cu) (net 11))
 (segment (start 46.355 66.675) (end 46.355 67.31) (width 0.381) (layer B.Cu) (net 23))
 (segment (start 46.99 67.945) (end 47.625 67.945) (width 0.381) (layer B.Cu) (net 23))
 (segment (start 46.355 67.31) (end 46.99 67.945) (width 0.381) (layer B.Cu) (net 23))
 (segment (start 44.45 55.88) (end 45.72 55.88) (width 0.381) (layer B.Cu) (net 23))
 (segment (start 52.07 68.58) (end 52.07 69.85) (width 0.381) (layer B.Cu) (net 23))
 (segment (start 47.625 67.945) (end 51.435 67.945) (width 0.381) (layer B.Cu) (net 23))
 (segment (start 51.435 67.945) (end 52.07 68.58) (width 0.381) (layer B.Cu) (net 23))
 (segment (start 46.355 56.515) (end 46.355 66.675) (width 0.381) (layer B.Cu) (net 23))
 (segment (start 45.72 55.88) (end 46.355 56.515) (width 0.381) (layer B.Cu) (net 23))
 (segment (start 72.39 65.0875) (end 55.5625 65.0875) (width 1.016) (layer F.Cu) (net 12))
 (segment (start 54.61 66.04) (end 54.61 69.85) (width 1.016) (layer F.Cu) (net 12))
 (segment (start 55.5625 65.0875) (end 54.61 66.04) (width 1.016) (layer F.Cu) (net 12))
 (segment (start 72.39 65.0875) (end 76.5175 65.0875) (width 1.016) (layer F.Cu) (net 12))
 (segment (start 76.5175 65.0875) (end 77.47 66.04) (width 1.016) (layer F.Cu) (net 12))
 (segment (start 52.07 77.47) (end 52.07 76.2) (width 0.381) (layer F.Cu) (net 18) (status 400000))
 (segment (start 47.625 76.2) (end 44.45 76.2) (width 0.381) (layer F.Cu) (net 18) (status 800000))
 (segment (start 48.26 75.565) (end 47.625 76.2) (width 0.381) (layer F.Cu) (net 18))
 (segment (start 51.435 75.565) (end 48.26 75.565) (width 0.381) (layer F.Cu) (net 18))
 (segment (start 52.07 76.2) (end 51.435 75.565) (width 0.381) (layer F.Cu) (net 18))
 (segment (start 72.39 82.2325) (end 55.5625 82.2325) (width 1.016) (layer F.Cu) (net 13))
 (segment (start 54.61 81.28) (end 54.61 77.47) (width 1.016) (layer F.Cu) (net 13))
 (segment (start 55.5625 82.2325) (end 54.61 81.28) (width 1.016) (layer F.Cu) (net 13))
 (segment (start 72.39 82.2325) (end 76.5175 82.2325) (width 1.016) (layer F.Cu) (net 13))
 (segment (start 76.5175 82.2325) (end 77.47 81.28) (width 1.016) (layer F.Cu) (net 13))
 (segment (start 64.77 77.47) (end 64.77 78.105) (width 0.381) (layer F.Cu) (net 19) (status C00000))
 (segment (start 45.085 74.295) (end 44.45 73.66) (width 0.381) (layer F.Cu) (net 19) (status 800000))
 (segment (start 59.69 74.295) (end 45.085 74.295) (width 0.381) (layer F.Cu) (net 19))
 (segment (start 60.96 75.565) (end 59.69 74.295) (width 0.381) (layer F.Cu) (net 19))
 (segment (start 60.96 78.105) (end 60.96 75.565) (width 0.381) (layer F.Cu) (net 19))
 (segment (start 61.595 78.74) (end 60.96 78.105) (width 0.381) (layer F.Cu) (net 19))
 (segment (start 64.135 78.74) (end 61.595 78.74) (width 0.381) (layer F.Cu) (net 19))
 (segment (start 64.77 78.105) (end 64.135 78.74) (width 0.381) (layer F.Cu) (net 19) (status 400000))
 (segment (start 72.39 75.2475) (end 63.1825 75.2475) (width 1.016) (layer F.Cu) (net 14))
 (segment (start 62.23 76.2) (end 62.23 77.47) (width 1.016) (layer F.Cu) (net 14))
 (segment (start 63.1825 75.2475) (end 62.23 76.2) (width 1.016) (layer F.Cu) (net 14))
 (segment (start 72.39 75.2475) (end 76.5175 75.2475) (width 1.016) (layer F.Cu) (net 14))
 (segment (start 76.5175 75.2475) (end 77.47 76.2) (width 1.016) (layer F.Cu) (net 14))
 (segment (start 38.1 80.645) (end 38.1 44.45) (width 0.381) (layer B.Cu) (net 17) (status 400000))
 (segment (start 38.1 44.45) (end 36.83 43.18) (width 0.381) (layer B.Cu) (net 17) (status 800000))
 (segment (start 40.64 80.645) (end 40.64 66.04) (width 0.381) (layer B.Cu) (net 22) (status 400000))
 (segment (start 40.64 66.04) (end 44.45 66.04) (width 0.381) (layer F.Cu) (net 22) (status 800000))
 (via (at 40.64 66.04) (size 0.889) (layers F.Cu B.Cu) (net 22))
 (segment (start 36.83 60.96) (end 41.91 60.96) (width 0.381) (layer F.Cu) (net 1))
 (via (at 41.91 60.96) (size 0.889) (layers F.Cu B.Cu) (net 1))
 (segment (start 41.91 60.96) (end 44.45 58.42) (width 0.381) (layer B.Cu) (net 1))
 (segment (start 57.15 49.53) (end 57.15 57.15) (width 1.016) (layer F.Cu) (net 1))
 (segment (start 57.15 49.53) (end 59.69 49.53) (width 1.016) (layer F.Cu) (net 1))
 (segment (start 57.15 57.15) (end 59.69 57.15) (width 1.016) (layer F.Cu) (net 1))
 (segment (start 72.39 80.3275) (end 60.6425 80.3275) (width 0.381) (layer F.Cu) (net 1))
 (segment (start 59.69 79.375) (end 59.69 77.47) (width 0.381) (layer F.Cu) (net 1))
 (segment (start 60.6425 80.3275) (end 59.69 79.375) (width 0.381) (layer F.Cu) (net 1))
 (segment (start 72.39 66.9925) (end 60.6425 66.9925) (width 0.381) (layer F.Cu) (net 1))
 (segment (start 59.69 67.945) (end 59.69 69.85) (width 0.381) (layer F.Cu) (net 1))
 (segment (start 60.6425 66.9925) (end 59.69 67.945) (width 0.381) (layer F.Cu) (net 1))
 (segment (start 72.39 60.0075) (end 60.6425 60.0075) (width 0.381) (layer F.Cu) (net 1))
 (segment (start 60.6425 60.0075) (end 59.69 59.055) (width 0.381) (layer F.Cu) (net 1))
 (segment (start 59.69 59.055) (end 59.69 57.15) (width 0.381) (layer F.Cu) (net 1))
 (segment (start 72.39 46.6725) (end 60.6425 46.6725) (width 0.381) (layer F.Cu) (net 1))
 (segment (start 59.69 47.625) (end 59.69 49.53) (width 0.381) (layer F.Cu) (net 1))
 (segment (start 60.6425 46.6725) (end 59.69 47.625) (width 0.381) (layer F.Cu) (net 1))
 (segment (start 72.39 49.8475) (end 72.39 46.6725) (width 0.381) (layer F.Cu) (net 1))
 (segment (start 72.39 60.0075) (end 72.39 56.8325) (width 0.381) (layer F.Cu) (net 1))
 (segment (start 72.39 66.9925) (end 72.39 70.1675) (width 0.381) (layer F.Cu) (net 1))
 (segment (start 72.39 77.1525) (end 72.39 80.3275) (width 0.381) (layer F.Cu) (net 1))
 (segment (start 57.15 77.47) (end 59.69 77.47) (width 1.016) (layer F.Cu) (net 1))
 (segment (start 59.69 69.85) (end 57.15 69.85) (width 1.016) (layer F.Cu) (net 1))
 (segment (start 44.45 60.96) (end 44.45 63.5) (width 0.381) (layer F.Cu) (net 16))
 (segment (start 36.83 58.42) (end 41.91 58.42) (width 0.381) (layer F.Cu) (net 16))
 (segment (start 41.91 58.42) (end 44.45 60.96) (width 0.381) (layer F.Cu) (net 16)))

